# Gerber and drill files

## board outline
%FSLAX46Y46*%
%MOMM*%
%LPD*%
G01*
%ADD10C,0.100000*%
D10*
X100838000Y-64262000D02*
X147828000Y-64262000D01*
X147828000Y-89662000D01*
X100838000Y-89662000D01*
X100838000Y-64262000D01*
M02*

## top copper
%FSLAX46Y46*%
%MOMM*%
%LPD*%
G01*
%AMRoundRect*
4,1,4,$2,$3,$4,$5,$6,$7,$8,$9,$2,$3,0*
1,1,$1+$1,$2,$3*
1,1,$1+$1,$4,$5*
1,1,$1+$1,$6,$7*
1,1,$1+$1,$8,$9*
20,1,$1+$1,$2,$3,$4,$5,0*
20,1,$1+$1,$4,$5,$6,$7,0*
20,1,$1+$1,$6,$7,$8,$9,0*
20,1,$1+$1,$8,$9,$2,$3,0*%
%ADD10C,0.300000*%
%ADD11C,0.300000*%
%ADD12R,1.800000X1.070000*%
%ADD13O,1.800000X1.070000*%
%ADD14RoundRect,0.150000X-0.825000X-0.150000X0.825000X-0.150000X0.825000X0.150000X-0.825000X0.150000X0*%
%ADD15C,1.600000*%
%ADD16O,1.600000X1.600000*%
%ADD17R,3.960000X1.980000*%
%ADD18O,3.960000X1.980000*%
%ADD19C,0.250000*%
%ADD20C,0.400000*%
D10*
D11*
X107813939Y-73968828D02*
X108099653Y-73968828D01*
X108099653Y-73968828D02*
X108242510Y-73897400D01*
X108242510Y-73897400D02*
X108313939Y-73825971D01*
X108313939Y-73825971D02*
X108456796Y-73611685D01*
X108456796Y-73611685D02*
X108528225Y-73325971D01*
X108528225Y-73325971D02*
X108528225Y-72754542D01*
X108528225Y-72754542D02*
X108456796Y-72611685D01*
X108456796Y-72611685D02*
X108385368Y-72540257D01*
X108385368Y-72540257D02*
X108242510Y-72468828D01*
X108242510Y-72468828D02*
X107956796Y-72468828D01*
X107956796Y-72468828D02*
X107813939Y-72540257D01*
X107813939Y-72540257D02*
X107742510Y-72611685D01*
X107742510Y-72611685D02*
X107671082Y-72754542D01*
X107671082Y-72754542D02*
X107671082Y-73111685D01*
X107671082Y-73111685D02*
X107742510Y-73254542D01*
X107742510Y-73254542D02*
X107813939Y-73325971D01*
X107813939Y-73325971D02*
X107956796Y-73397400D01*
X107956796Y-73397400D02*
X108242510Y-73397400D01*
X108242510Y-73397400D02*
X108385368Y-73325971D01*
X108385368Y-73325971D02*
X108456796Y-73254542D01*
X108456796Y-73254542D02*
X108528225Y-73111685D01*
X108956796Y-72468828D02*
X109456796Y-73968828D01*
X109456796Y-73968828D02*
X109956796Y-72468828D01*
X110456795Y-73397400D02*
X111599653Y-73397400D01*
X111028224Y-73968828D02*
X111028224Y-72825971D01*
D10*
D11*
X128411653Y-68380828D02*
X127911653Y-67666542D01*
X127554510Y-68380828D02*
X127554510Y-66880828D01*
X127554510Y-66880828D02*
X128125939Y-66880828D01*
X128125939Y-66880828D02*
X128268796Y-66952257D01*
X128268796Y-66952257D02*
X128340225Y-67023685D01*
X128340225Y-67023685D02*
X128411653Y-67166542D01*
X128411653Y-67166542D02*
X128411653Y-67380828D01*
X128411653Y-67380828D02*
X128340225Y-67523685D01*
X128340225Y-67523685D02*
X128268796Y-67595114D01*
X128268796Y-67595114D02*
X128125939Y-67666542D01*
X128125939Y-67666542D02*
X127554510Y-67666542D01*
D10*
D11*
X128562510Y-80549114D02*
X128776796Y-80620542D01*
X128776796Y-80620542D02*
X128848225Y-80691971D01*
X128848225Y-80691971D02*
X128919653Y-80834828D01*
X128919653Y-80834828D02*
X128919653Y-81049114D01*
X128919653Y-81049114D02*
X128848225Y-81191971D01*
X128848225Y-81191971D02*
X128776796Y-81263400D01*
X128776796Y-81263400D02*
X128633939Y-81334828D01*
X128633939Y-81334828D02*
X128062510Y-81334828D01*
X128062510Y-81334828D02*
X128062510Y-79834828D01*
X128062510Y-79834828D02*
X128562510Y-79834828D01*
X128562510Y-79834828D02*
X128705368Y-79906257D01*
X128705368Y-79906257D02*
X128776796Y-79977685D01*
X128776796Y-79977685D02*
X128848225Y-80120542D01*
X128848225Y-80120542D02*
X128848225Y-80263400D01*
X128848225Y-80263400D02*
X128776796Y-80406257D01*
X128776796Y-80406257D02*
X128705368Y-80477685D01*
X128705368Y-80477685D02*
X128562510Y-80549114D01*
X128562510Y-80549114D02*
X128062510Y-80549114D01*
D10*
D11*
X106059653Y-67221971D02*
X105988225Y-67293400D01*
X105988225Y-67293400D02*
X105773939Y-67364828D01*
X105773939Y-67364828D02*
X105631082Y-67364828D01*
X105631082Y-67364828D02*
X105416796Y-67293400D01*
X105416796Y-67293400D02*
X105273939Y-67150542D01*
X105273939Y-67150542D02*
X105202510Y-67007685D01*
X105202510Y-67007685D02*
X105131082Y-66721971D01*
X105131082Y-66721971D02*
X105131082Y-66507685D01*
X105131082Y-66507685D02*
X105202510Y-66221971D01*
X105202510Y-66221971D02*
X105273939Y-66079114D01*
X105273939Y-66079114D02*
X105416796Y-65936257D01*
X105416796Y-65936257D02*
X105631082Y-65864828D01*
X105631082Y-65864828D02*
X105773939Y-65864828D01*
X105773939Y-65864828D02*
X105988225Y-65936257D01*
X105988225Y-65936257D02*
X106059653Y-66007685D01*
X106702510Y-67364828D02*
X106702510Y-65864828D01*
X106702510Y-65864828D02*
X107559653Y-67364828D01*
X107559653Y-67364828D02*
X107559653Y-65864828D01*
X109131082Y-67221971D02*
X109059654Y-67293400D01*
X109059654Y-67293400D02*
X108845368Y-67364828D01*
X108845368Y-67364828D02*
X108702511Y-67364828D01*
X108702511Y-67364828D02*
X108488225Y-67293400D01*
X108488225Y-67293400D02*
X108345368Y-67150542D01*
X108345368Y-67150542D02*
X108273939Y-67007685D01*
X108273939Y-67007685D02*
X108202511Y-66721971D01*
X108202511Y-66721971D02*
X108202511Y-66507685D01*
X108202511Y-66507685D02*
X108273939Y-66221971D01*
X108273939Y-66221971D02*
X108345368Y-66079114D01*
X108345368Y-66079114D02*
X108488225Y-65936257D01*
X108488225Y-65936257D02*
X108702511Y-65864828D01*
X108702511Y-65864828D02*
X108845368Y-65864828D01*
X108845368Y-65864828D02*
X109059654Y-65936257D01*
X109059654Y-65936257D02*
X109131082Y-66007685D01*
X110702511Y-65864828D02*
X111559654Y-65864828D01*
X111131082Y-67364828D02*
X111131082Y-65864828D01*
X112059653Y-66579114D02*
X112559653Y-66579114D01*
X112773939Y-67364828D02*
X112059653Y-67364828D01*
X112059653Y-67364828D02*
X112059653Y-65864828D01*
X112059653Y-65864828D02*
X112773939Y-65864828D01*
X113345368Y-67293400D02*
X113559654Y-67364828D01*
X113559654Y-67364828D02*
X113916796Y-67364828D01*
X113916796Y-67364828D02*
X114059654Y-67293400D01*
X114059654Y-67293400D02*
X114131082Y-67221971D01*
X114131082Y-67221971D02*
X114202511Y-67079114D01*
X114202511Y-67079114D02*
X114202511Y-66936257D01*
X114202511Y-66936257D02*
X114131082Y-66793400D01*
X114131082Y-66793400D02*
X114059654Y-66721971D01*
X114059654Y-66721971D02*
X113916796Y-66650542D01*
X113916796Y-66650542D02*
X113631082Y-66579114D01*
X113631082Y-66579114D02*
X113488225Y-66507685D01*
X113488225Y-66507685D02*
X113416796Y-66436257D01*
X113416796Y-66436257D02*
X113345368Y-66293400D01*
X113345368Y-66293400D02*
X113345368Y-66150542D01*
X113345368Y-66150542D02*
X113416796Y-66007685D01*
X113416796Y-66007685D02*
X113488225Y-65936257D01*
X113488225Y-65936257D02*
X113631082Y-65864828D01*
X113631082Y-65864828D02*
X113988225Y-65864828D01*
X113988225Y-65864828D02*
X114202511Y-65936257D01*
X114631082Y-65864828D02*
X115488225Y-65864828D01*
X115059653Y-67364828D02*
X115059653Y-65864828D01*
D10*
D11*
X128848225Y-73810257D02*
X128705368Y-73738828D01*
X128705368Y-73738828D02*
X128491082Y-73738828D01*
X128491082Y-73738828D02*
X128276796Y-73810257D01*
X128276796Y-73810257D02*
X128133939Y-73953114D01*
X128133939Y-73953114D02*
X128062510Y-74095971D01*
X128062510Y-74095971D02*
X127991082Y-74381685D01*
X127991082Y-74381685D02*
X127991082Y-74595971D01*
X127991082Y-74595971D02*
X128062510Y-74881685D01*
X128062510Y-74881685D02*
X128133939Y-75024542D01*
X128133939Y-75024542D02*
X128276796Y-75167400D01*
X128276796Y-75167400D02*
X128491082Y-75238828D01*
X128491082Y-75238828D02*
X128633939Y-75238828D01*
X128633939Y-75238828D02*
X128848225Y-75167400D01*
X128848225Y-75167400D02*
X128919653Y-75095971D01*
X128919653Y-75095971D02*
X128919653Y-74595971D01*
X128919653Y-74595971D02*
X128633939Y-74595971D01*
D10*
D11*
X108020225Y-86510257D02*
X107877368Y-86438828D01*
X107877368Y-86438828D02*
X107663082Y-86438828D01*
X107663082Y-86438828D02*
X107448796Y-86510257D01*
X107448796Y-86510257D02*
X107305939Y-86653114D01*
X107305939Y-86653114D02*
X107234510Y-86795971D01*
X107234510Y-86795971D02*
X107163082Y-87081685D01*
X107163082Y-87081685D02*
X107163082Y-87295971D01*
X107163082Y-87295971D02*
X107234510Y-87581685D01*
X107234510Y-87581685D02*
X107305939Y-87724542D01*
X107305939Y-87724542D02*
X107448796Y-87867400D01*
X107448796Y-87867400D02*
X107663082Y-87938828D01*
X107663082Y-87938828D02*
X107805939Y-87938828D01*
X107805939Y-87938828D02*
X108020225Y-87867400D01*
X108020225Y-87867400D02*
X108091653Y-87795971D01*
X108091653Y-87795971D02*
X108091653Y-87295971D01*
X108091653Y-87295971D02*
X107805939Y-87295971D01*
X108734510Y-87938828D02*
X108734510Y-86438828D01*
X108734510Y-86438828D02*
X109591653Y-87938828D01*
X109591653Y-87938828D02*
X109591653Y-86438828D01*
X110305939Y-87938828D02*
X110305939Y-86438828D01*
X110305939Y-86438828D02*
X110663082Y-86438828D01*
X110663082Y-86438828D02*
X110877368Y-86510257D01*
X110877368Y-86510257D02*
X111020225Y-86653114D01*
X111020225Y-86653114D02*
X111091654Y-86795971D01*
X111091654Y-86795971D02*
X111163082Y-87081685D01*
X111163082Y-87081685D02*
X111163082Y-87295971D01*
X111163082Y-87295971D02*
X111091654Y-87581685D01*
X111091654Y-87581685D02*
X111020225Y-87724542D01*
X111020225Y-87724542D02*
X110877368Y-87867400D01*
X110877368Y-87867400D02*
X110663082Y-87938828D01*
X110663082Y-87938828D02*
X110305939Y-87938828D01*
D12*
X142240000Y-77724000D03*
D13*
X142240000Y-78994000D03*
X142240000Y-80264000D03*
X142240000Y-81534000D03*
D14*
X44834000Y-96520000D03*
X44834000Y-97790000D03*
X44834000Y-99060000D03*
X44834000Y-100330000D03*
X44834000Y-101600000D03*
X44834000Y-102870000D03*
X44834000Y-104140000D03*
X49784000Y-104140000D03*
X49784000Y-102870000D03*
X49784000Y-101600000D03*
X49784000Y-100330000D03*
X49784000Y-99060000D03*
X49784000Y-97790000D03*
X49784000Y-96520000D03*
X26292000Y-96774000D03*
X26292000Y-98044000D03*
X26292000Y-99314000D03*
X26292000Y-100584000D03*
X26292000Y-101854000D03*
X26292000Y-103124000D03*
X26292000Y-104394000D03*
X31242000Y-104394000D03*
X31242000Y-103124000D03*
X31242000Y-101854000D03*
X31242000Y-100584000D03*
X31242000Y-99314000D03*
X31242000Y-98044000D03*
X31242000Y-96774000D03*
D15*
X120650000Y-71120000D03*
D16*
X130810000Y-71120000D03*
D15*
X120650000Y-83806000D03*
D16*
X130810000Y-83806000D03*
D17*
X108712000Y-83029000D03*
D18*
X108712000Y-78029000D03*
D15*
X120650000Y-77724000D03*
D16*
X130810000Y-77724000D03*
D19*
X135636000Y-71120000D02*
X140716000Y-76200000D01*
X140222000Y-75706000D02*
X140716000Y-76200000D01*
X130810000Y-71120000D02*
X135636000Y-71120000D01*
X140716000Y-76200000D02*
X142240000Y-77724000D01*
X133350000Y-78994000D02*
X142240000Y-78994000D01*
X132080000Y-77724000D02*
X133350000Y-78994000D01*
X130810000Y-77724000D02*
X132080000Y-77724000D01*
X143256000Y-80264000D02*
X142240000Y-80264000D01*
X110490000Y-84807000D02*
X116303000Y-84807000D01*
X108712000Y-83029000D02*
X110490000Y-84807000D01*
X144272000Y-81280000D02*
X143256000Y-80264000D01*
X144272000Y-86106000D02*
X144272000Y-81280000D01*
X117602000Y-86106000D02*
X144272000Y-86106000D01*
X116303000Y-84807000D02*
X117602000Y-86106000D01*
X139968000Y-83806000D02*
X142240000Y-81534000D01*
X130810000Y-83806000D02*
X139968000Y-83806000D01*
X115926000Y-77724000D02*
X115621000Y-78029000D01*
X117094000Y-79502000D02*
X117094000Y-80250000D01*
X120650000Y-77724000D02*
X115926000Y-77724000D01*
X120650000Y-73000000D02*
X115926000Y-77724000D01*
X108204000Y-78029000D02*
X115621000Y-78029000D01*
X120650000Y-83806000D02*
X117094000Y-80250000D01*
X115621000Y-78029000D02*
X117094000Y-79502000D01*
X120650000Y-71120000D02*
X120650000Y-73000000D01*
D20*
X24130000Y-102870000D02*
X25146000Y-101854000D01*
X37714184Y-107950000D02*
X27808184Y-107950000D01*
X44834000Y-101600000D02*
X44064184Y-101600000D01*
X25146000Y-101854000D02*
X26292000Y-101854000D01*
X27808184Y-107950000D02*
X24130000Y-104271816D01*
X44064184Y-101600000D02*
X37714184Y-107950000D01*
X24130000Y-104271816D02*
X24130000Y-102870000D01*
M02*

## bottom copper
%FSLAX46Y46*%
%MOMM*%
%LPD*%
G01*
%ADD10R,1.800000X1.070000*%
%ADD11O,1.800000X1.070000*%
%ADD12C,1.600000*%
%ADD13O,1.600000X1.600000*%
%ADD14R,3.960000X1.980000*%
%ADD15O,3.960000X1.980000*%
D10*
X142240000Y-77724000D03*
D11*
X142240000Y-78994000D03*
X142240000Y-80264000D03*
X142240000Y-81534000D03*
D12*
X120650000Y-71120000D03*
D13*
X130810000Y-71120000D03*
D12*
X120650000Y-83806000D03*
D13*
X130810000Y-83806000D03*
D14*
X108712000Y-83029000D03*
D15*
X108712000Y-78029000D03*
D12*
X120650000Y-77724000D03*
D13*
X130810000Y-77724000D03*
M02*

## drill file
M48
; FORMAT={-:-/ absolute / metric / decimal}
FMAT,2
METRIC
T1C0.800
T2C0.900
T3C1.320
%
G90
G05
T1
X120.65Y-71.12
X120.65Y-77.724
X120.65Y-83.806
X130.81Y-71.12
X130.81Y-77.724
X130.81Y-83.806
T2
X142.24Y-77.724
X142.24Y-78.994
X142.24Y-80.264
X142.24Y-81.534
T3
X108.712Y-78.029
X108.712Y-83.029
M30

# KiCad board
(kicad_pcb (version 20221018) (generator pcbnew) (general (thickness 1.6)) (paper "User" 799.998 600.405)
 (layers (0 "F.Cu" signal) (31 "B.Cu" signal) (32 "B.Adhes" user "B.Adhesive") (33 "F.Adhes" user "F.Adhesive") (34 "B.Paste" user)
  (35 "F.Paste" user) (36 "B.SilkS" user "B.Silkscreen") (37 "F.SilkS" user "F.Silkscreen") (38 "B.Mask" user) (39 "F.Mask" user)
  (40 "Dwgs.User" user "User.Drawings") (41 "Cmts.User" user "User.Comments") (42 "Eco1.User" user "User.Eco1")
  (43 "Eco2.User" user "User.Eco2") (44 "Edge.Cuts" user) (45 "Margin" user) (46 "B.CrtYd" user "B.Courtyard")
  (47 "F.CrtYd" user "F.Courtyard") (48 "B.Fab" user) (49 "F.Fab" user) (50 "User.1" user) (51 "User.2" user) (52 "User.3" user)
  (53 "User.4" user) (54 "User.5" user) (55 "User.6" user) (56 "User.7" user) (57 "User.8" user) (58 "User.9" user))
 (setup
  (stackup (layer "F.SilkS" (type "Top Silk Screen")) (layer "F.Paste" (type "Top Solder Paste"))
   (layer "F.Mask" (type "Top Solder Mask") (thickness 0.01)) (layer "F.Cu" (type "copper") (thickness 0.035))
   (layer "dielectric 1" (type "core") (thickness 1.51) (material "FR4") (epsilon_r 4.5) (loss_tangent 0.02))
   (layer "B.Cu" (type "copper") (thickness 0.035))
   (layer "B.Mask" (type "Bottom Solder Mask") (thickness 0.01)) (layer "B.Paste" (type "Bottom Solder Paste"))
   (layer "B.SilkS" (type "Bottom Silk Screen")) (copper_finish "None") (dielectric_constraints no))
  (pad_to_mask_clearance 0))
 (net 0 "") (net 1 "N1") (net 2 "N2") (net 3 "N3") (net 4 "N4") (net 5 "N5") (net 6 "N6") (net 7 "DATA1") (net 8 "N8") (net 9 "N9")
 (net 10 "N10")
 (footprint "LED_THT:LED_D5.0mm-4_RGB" (layer "F.Cu") (at 142.24 77.724 -90)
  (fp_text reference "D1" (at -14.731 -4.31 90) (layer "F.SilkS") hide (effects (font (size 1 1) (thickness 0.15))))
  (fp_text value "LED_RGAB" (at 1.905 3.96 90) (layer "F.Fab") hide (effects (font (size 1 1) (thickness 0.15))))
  (pad "1" thru_hole rect (at 0 0 270) (size 1.07 1.8) (drill 0.9) (layers "*.Cu" "*.Mask") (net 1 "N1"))
  (pad "2" thru_hole oval (at 1.27 0 270) (size 1.07 1.8) (drill 0.9) (layers "*.Cu" "*.Mask") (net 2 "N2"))
  (pad "3" thru_hole oval (at 2.54 0 270) (size 1.07 1.8) (drill 0.9) (layers "*.Cu" "*.Mask") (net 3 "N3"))
  (pad "4" thru_hole oval (at 3.81 0 270) (size 1.07 1.8) (drill 0.9) (layers "*.Cu" "*.Mask") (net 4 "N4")))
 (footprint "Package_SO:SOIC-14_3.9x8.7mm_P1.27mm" (layer "F.Cu") (at 47.309 100.33)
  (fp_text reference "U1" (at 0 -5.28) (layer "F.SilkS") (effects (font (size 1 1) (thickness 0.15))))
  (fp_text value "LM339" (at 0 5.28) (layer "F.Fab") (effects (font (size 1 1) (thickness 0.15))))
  (pad "1" smd roundrect (at -2.475 -3.81) (size 1.95 0.6) (layers "F.Cu" "F.Paste" "F.Mask") (roundrect_rratio 0.25))
  (pad "2" smd roundrect (at -2.475 -2.54) (size 1.95 0.6) (layers "F.Cu" "F.Paste" "F.Mask") (roundrect_rratio 0.25) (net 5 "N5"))
  (pad "3" smd roundrect (at -2.475 -1.27) (size 1.95 0.6) (layers "F.Cu" "F.Paste" "F.Mask") (roundrect_rratio 0.25))
  (pad "4" smd roundrect (at -2.475 0) (size 1.95 0.6) (layers "F.Cu" "F.Paste" "F.Mask") (roundrect_rratio 0.25) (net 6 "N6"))
  (pad "5" smd roundrect (at -2.475 1.27) (size 1.95 0.6) (layers "F.Cu" "F.Paste" "F.Mask") (roundrect_rratio 0.25) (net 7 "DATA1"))
  (pad "6" smd roundrect (at -2.475 2.54) (size 1.95 0.6) (layers "F.Cu" "F.Paste" "F.Mask") (roundrect_rratio 0.25))
  (pad "7" smd roundrect (at -2.475 3.81) (size 1.95 0.6) (layers "F.Cu" "F.Paste" "F.Mask") (roundrect_rratio 0.25))
  (pad "8" smd roundrect (at 2.475 3.81) (size 1.95 0.6) (layers "F.Cu" "F.Paste" "F.Mask") (roundrect_rratio 0.25))
  (pad "9" smd roundrect (at 2.475 2.54) (size 1.95 0.6) (layers "F.Cu" "F.Paste" "F.Mask") (roundrect_rratio 0.25))
  (pad "10" smd roundrect (at 2.475 1.27) (size 1.95 0.6) (layers "F.Cu" "F.Paste" "F.Mask") (roundrect_rratio 0.25))
  (pad "11" smd roundrect (at 2.475 0) (size 1.95 0.6) (layers "F.Cu" "F.Paste" "F.Mask") (roundrect_rratio 0.25))
  (pad "12" smd roundrect (at 2.475 -1.27) (size 1.95 0.6) (layers "F.Cu" "F.Paste" "F.Mask") (roundrect_rratio 0.25))
  (pad "13" smd roundrect (at 2.475 -2.54) (size 1.95 0.6) (layers "F.Cu" "F.Paste" "F.Mask") (roundrect_rratio 0.25))
  (pad "14" smd roundrect (at 2.475 -3.81) (size 1.95 0.6) (layers "F.Cu" "F.Paste" "F.Mask") (roundrect_rratio 0.25)))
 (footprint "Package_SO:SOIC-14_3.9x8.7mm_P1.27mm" (layer "F.Cu") (at 28.767 100.584)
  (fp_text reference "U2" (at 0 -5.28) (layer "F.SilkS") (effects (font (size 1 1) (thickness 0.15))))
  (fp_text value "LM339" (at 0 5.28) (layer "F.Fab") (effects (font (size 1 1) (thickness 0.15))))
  (pad "1" smd roundrect (at -2.475 -3.81) (size 1.95 0.6) (layers "F.Cu" "F.Paste" "F.Mask") (roundrect_rratio 0.25))
  (pad "2" smd roundrect (at -2.475 -2.54) (size 1.95 0.6) (layers "F.Cu" "F.Paste" "F.Mask") (roundrect_rratio 0.25) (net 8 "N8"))
  (pad "3" smd roundrect (at -2.475 -1.27) (size 1.95 0.6) (layers "F.Cu" "F.Paste" "F.Mask") (roundrect_rratio 0.25))
  (pad "4" smd roundrect (at -2.475 0) (size 1.95 0.6) (layers "F.Cu" "F.Paste" "F.Mask") (roundrect_rratio 0.25) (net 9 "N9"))
  (pad "5" smd roundrect (at -2.475 1.27) (size 1.95 0.6) (layers "F.Cu" "F.Paste" "F.Mask") (roundrect_rratio 0.25) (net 7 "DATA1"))
  (pad "6" smd roundrect (at -2.475 2.54) (size 1.95 0.6) (layers "F.Cu" "F.Paste" "F.Mask") (roundrect_rratio 0.25))
  (pad "7" smd roundrect (at -2.475 3.81) (size 1.95 0.6) (layers "F.Cu" "F.Paste" "F.Mask") (roundrect_rratio 0.25))
  (pad "8" smd roundrect (at 2.475 3.81) (size 1.95 0.6) (layers "F.Cu" "F.Paste" "F.Mask") (roundrect_rratio 0.25))
  (pad "9" smd roundrect (at 2.475 2.54) (size 1.95 0.6) (layers "F.Cu" "F.Paste" "F.Mask") (roundrect_rratio 0.25))
  (pad "10" smd roundrect (at 2.475 1.27) (size 1.95 0.6) (layers "F.Cu" "F.Paste" "F.Mask") (roundrect_rratio 0.25))
  (pad "11" smd roundrect (at 2.475 0) (size 1.95 0.6) (layers "F.Cu" "F.Paste" "F.Mask") (roundrect_rratio 0.25))
  (pad "12" smd roundrect (at 2.475 -1.27) (size 1.95 0.6) (layers "F.Cu" "F.Paste" "F.Mask") (roundrect_rratio 0.25))
  (pad "13" smd roundrect (at 2.475 -2.54) (size 1.95 0.6) (layers "F.Cu" "F.Paste" "F.Mask") (roundrect_rratio 0.25))
  (pad "14" smd roundrect (at 2.475 -3.81) (size 1.95 0.6) (layers "F.Cu" "F.Paste" "F.Mask") (roundrect_rratio 0.25)))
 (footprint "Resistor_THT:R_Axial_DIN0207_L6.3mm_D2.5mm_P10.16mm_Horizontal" (layer "F.Cu") (at 120.65 71.12)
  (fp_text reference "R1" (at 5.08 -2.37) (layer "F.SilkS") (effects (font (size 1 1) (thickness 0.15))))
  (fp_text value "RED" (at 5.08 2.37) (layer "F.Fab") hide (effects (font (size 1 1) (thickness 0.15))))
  (pad "1" thru_hole circle (at 0 0) (size 1.6 1.6) (drill 0.8) (layers "*.Cu" "*.Mask") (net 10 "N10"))
  (pad "2" thru_hole oval (at 10.16 0) (size 1.6 1.6) (drill 0.8) (layers "*.Cu" "*.Mask") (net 1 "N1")))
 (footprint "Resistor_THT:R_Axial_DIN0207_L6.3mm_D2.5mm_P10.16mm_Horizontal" (layer "F.Cu") (at 120.65 83.806)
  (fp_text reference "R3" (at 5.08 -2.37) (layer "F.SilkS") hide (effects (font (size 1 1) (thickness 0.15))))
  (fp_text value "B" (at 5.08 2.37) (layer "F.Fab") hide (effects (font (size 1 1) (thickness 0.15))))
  (pad "1" thru_hole circle (at 0 0) (size 1.6 1.6) (drill 0.8) (layers "*.Cu" "*.Mask") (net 10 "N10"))
  (pad "2" thru_hole oval (at 10.16 0) (size 1.6 1.6) (drill 0.8) (layers "*.Cu" "*.Mask") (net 4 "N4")))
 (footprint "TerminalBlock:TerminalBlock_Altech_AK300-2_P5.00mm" (layer "F.Cu") (at 108.712 83.029 90)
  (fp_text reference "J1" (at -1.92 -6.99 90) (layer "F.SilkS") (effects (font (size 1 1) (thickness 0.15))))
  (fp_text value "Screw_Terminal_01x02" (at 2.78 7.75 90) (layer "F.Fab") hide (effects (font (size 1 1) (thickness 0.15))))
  (pad "1" thru_hole rect (at 0 0 90) (size 1.98 3.96) (drill 1.32) (layers "*.Cu" "*.Mask") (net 3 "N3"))
  (pad "2" thru_hole oval (at 5 0 90) (size 1.98 3.96) (drill 1.32) (layers "*.Cu" "*.Mask") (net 10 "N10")))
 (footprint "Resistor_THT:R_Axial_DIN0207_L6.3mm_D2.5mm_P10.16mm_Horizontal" (layer "F.Cu") (at 120.65 77.724)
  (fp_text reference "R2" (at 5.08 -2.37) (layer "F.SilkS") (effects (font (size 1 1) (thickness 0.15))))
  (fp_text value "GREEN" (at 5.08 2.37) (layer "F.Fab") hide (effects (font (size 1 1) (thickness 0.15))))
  (pad "1" thru_hole circle (at 0 0) (size 1.6 1.6) (drill 0.8) (layers "*.Cu" "*.Mask") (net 10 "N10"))
  (pad "2" thru_hole oval (at 10.16 0) (size 1.6 1.6) (drill 0.8) (layers "*.Cu" "*.Mask") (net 2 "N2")))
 (gr_rect (start 100.838 64.262) (end 147.828 89.662) (stroke (width 0.1) (type default)) (fill none) (layer "Edge.Cuts"))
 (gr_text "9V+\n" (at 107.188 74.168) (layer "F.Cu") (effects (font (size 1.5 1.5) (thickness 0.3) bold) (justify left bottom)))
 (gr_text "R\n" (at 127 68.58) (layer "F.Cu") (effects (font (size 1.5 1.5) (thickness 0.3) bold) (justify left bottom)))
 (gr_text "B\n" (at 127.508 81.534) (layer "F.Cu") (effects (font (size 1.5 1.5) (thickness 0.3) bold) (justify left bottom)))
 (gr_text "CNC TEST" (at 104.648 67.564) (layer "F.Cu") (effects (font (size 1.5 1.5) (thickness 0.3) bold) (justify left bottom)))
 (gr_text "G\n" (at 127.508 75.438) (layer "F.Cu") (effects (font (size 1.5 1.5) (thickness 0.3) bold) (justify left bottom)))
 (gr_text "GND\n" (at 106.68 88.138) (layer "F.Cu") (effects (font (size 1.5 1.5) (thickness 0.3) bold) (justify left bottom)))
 (segment (start 135.636 71.12) (end 140.716 76.2) (width 0.25) (layer "F.Cu") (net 1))
 (segment (start 140.222 75.706) (end 140.716 76.2) (width 0.25) (layer "F.Cu") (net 1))
 (segment (start 130.81 71.12) (end 135.636 71.12) (width 0.25) (layer "F.Cu") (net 1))
 (segment (start 140.716 76.2) (end 142.24 77.724) (width 0.25) (layer "F.Cu") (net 1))
 (segment (start 133.35 78.994) (end 142.24 78.994) (width 0.25) (layer "F.Cu") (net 2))
 (segment (start 132.08 77.724) (end 133.35 78.994) (width 0.25) (layer "F.Cu") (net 2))
 (segment (start 130.81 77.724) (end 132.08 77.724) (width 0.25) (layer "F.Cu") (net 2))
 (segment (start 143.256 80.264) (end 142.24 80.264) (width 0.25) (layer "F.Cu") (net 3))
 (segment (start 110.49 84.807) (end 116.303 84.807) (width 0.25) (layer "F.Cu") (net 3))
 (segment (start 108.712 83.029) (end 110.49 84.807) (width 0.25) (layer "F.Cu") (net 3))
 (segment (start 144.272 81.28) (end 143.256 80.264) (width 0.25) (layer "F.Cu") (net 3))
 (segment (start 144.272 86.106) (end 144.272 81.28) (width 0.25) (layer "F.Cu") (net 3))
 (segment (start 117.602 86.106) (end 144.272 86.106) (width 0.25) (layer "F.Cu") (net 3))
 (segment (start 116.303 84.807) (end 117.602 86.106) (width 0.25) (layer "F.Cu") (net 3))
 (segment (start 139.968 83.806) (end 142.24 81.534) (width 0.25) (layer "F.Cu") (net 4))
 (segment (start 130.81 83.806) (end 139.968 83.806) (width 0.25) (layer "F.Cu") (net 4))
 (segment (start 115.926 77.724) (end 115.621 78.029) (width 0.25) (layer "F.Cu") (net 10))
 (segment (start 117.094 79.502) (end 117.094 80.25) (width 0.25) (layer "F.Cu") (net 10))
 (segment (start 120.65 77.724) (end 115.926 77.724) (width 0.25) (layer "F.Cu") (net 10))
 (segment (start 120.65 73) (end 115.926 77.724) (width 0.25) (layer "F.Cu") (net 10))
 (segment (start 108.204 78.029) (end 115.621 78.029) (width 0.25) (layer "F.Cu") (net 10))
 (segment (start 120.65 83.806) (end 117.094 80.25) (width 0.25) (layer "F.Cu") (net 10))
 (segment (start 115.621 78.029) (end 117.094 79.502) (width 0.25) (layer "F.Cu") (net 10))
 (segment (start 120.65 71.12) (end 120.65 73) (width 0.25) (layer "F.Cu") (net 10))
 (segment (start 24.13 102.87) (end 25.146 101.854) (width 0.4) (layer "F.Cu") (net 7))
 (segment (start 37.714184 107.95) (end 27.808184 107.95) (width 0.4) (layer "F.Cu") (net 7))
 (segment (start 44.834 101.6) (end 44.064184 101.6) (width 0.4) (layer "F.Cu") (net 7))
 (segment (start 25.146 101.854) (end 26.292 101.854) (width 0.4) (layer "F.Cu") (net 7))
 (segment (start 27.808184 107.95) (end 24.13 104.271816) (width 0.4) (layer "F.Cu") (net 7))
 (segment (start 44.064184 101.6) (end 37.714184 107.95) (width 0.4) (layer "F.Cu") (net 7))
 (segment (start 24.13 104.271816) (end 24.13 102.87) (width 0.4) (layer "F.Cu") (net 7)))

